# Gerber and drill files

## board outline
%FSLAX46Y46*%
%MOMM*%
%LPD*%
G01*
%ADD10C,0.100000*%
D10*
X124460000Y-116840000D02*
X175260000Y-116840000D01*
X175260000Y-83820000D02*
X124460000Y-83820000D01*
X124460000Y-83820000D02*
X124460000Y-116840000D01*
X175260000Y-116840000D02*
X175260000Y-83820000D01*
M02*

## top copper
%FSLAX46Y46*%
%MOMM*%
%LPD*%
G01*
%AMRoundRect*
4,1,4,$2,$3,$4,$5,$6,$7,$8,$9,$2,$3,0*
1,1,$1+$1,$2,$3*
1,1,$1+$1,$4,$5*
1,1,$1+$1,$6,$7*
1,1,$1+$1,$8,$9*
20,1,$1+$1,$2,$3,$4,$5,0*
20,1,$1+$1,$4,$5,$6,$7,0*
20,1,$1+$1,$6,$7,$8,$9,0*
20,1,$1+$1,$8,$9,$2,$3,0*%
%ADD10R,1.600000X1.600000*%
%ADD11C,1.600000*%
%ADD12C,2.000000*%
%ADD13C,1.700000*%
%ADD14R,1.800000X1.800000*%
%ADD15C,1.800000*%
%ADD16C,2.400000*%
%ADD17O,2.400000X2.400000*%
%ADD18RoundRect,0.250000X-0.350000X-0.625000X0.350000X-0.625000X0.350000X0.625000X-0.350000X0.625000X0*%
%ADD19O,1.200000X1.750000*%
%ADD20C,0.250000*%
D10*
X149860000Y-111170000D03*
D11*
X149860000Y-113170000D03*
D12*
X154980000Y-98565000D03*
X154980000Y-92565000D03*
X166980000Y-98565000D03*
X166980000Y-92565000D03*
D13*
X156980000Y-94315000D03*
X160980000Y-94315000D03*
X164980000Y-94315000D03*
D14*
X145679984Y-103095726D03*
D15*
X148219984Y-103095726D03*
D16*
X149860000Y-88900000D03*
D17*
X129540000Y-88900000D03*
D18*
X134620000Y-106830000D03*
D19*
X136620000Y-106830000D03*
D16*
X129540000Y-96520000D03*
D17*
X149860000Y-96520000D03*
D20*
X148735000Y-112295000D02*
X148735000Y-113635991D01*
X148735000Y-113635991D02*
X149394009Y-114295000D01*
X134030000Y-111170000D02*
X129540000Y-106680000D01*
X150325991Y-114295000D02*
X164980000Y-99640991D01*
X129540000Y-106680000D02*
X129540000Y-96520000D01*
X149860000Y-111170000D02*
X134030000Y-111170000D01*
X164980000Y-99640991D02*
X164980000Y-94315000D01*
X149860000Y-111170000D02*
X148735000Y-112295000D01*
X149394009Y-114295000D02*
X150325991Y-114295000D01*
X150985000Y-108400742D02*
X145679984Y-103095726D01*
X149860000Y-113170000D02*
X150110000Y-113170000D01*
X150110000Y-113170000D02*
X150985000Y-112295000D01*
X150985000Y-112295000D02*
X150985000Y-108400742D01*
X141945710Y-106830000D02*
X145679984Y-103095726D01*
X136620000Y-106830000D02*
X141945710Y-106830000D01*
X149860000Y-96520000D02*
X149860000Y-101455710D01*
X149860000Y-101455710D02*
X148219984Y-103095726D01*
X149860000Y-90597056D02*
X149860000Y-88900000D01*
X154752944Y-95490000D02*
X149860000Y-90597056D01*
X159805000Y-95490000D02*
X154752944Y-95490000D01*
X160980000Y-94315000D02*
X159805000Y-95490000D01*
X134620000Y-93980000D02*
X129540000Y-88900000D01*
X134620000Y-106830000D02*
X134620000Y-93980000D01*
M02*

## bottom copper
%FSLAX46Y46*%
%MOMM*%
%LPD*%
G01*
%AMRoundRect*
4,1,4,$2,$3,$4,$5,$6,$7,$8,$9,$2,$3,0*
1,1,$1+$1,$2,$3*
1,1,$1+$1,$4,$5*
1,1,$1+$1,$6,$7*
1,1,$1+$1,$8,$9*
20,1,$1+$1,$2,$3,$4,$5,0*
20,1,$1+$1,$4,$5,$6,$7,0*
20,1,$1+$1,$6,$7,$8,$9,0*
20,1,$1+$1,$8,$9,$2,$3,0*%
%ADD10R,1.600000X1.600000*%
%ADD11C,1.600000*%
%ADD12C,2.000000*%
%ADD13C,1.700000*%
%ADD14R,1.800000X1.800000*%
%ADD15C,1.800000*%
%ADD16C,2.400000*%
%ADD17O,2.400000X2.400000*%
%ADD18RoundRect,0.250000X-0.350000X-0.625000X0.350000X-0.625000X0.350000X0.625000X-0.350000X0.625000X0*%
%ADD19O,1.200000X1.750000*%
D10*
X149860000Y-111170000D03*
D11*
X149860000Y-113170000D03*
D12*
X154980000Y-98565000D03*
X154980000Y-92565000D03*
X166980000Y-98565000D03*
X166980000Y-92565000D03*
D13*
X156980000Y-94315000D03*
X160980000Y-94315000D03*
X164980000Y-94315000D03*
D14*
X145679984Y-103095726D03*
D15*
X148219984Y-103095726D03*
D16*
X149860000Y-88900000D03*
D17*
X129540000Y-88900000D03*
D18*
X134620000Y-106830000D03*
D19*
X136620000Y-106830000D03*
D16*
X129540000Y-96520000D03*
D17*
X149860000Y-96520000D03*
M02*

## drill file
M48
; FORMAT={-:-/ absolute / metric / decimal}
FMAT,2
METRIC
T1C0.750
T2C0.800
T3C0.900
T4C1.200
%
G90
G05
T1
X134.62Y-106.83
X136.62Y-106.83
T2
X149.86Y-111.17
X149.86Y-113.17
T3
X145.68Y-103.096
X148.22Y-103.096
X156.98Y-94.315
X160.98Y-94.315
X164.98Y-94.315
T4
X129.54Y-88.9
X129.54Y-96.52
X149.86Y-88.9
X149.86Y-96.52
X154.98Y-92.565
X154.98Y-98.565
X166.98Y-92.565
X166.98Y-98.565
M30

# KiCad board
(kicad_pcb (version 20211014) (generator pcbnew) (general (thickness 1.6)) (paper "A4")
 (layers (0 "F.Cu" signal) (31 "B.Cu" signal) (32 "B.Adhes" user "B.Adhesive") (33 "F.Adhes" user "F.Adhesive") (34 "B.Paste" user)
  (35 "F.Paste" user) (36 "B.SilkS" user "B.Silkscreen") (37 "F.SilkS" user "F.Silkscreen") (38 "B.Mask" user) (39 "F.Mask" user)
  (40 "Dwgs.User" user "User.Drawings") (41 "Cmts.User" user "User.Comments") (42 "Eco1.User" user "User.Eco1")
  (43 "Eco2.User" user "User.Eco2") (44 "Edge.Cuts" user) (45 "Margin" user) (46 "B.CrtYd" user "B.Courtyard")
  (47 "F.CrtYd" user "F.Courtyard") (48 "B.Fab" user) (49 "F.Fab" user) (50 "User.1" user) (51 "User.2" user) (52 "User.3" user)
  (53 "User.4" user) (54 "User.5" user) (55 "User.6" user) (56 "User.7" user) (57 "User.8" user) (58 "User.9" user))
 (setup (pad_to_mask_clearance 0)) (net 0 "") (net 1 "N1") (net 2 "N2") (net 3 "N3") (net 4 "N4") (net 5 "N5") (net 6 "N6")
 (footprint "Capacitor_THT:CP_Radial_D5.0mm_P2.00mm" (layer "F.Cu") (at 149.86 111.17 -90)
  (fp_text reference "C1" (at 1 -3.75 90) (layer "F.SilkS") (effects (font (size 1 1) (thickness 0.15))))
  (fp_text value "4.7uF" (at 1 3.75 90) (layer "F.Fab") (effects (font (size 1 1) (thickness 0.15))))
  (pad "1" thru_hole rect (at 0 0 270) (size 1.6 1.6) (drill 0.8) (layers *.Cu *.Mask) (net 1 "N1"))
  (pad "2" thru_hole circle (at 2 0 270) (size 1.6 1.6) (drill 0.8) (layers *.Cu *.Mask) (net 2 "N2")))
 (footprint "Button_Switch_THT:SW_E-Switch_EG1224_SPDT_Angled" (layer "F.Cu") (at 156.98 94.315)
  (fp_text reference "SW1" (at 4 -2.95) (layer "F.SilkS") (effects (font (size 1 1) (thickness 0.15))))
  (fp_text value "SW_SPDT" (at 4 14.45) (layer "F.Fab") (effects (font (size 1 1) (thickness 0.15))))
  (pad "" thru_hole circle (at -2 4.25) (size 2 2) (drill 1.2) (layers *.Cu *.Mask))
  (pad "" thru_hole circle (at -2 -1.75) (size 2 2) (drill 1.2) (layers *.Cu *.Mask))
  (pad "" thru_hole circle (at 10 4.25) (size 2 2) (drill 1.2) (layers *.Cu *.Mask))
  (pad "" thru_hole circle (at 10 -1.75) (size 2 2) (drill 1.2) (layers *.Cu *.Mask))
  (pad "1" thru_hole circle (at 0 0) (size 1.7 1.7) (drill 0.9) (layers *.Cu *.Mask) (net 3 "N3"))
  (pad "2" thru_hole circle (at 4 0) (size 1.7 1.7) (drill 0.9) (layers *.Cu *.Mask) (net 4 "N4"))
  (pad "3" thru_hole circle (at 8 0) (size 1.7 1.7) (drill 0.9) (layers *.Cu *.Mask) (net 1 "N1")))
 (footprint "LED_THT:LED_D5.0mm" (layer "F.Cu") (at 145.679984 103.095726)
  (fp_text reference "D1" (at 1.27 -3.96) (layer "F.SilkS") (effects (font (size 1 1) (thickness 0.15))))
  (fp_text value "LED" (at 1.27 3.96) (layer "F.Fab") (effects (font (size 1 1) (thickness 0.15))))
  (pad "1" thru_hole rect (at 0 0) (size 1.8 1.8) (drill 0.9) (layers *.Cu *.Mask) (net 2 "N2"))
  (pad "2" thru_hole circle (at 2.54 0) (size 1.8 1.8) (drill 0.9) (layers *.Cu *.Mask) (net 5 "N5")))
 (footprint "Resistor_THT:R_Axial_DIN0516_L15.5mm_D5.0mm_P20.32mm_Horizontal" (layer "F.Cu") (at 149.86 88.9 180)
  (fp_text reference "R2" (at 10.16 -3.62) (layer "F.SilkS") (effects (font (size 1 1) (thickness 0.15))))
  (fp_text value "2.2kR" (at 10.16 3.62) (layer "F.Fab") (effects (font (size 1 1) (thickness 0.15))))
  (pad "1" thru_hole circle (at 0 0 180) (size 2.4 2.4) (drill 1.2) (layers *.Cu *.Mask) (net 4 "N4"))
  (pad "2" thru_hole oval (at 20.32 0 180) (size 2.4 2.4) (drill 1.2) (layers *.Cu *.Mask) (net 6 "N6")))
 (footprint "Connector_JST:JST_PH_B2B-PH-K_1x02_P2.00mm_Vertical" (layer "F.Cu") (at 134.62 106.83)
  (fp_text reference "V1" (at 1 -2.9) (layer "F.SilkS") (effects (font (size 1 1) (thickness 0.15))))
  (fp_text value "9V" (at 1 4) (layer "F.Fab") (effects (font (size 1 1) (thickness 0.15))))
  (pad "1" thru_hole roundrect (at 0 0) (size 1.2 1.75) (drill 0.75) (layers *.Cu *.Mask) (roundrect_rratio 0.208333) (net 6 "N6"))
  (pad "2" thru_hole oval (at 2 0) (size 1.2 1.75) (drill 0.75) (layers *.Cu *.Mask) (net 2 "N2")))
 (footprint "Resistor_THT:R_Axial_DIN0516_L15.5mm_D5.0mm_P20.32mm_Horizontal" (layer "F.Cu") (at 129.54 96.52)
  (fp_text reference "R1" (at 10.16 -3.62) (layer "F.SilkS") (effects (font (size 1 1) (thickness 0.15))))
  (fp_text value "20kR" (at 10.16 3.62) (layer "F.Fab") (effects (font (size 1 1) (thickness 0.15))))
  (pad "1" thru_hole circle (at 0 0) (size 2.4 2.4) (drill 1.2) (layers *.Cu *.Mask) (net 1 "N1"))
  (pad "2" thru_hole oval (at 20.32 0) (size 2.4 2.4) (drill 1.2) (layers *.Cu *.Mask) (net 5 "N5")))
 (gr_line (start 124.46 116.84) (end 175.26 116.84) (layer "Edge.Cuts") (width 0.1))
 (gr_line (start 175.26 83.82) (end 124.46 83.82) (layer "Edge.Cuts") (width 0.1))
 (gr_line (start 124.46 83.82) (end 124.46 116.84) (layer "Edge.Cuts") (width 0.1))
 (gr_line (start 175.26 116.84) (end 175.26 83.82) (layer "Edge.Cuts") (width 0.1))
 (segment (start 148.735 112.295) (end 148.735 113.635991) (width 0.25) (layer "F.Cu") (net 1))
 (segment (start 148.735 113.635991) (end 149.394009 114.295) (width 0.25) (layer "F.Cu") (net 1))
 (segment (start 134.03 111.17) (end 129.54 106.68) (width 0.25) (layer "F.Cu") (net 1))
 (segment (start 150.325991 114.295) (end 164.98 99.640991) (width 0.25) (layer "F.Cu") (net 1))
 (segment (start 129.54 106.68) (end 129.54 96.52) (width 0.25) (layer "F.Cu") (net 1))
 (segment (start 149.86 111.17) (end 134.03 111.17) (width 0.25) (layer "F.Cu") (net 1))
 (segment (start 164.98 99.640991) (end 164.98 94.315) (width 0.25) (layer "F.Cu") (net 1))
 (segment (start 149.86 111.17) (end 148.735 112.295) (width 0.25) (layer "F.Cu") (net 1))
 (segment (start 149.394009 114.295) (end 150.325991 114.295) (width 0.25) (layer "F.Cu") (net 1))
 (segment (start 150.985 108.400742) (end 145.679984 103.095726) (width 0.25) (layer "F.Cu") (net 2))
 (segment (start 149.86 113.17) (end 150.11 113.17) (width 0.25) (layer "F.Cu") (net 2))
 (segment (start 150.11 113.17) (end 150.985 112.295) (width 0.25) (layer "F.Cu") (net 2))
 (segment (start 150.985 112.295) (end 150.985 108.400742) (width 0.25) (layer "F.Cu") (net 2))
 (segment (start 141.94571 106.83) (end 145.679984 103.095726) (width 0.25) (layer "F.Cu") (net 2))
 (segment (start 136.62 106.83) (end 141.94571 106.83) (width 0.25) (layer "F.Cu") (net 2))
 (segment (start 149.86 96.52) (end 149.86 101.45571) (width 0.25) (layer "F.Cu") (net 5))
 (segment (start 149.86 101.45571) (end 148.219984 103.095726) (width 0.25) (layer "F.Cu") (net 5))
 (segment (start 149.86 90.597056) (end 149.86 88.9) (width 0.25) (layer "F.Cu") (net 4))
 (segment (start 154.752944 95.49) (end 149.86 90.597056) (width 0.25) (layer "F.Cu") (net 4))
 (segment (start 159.805 95.49) (end 154.752944 95.49) (width 0.25) (layer "F.Cu") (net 4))
 (segment (start 160.98 94.315) (end 159.805 95.49) (width 0.25) (layer "F.Cu") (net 4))
 (segment (start 134.62 93.98) (end 129.54 88.9) (width 0.25) (layer "F.Cu") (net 6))
 (segment (start 134.62 106.83) (end 134.62 93.98) (width 0.25) (layer "F.Cu") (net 6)))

